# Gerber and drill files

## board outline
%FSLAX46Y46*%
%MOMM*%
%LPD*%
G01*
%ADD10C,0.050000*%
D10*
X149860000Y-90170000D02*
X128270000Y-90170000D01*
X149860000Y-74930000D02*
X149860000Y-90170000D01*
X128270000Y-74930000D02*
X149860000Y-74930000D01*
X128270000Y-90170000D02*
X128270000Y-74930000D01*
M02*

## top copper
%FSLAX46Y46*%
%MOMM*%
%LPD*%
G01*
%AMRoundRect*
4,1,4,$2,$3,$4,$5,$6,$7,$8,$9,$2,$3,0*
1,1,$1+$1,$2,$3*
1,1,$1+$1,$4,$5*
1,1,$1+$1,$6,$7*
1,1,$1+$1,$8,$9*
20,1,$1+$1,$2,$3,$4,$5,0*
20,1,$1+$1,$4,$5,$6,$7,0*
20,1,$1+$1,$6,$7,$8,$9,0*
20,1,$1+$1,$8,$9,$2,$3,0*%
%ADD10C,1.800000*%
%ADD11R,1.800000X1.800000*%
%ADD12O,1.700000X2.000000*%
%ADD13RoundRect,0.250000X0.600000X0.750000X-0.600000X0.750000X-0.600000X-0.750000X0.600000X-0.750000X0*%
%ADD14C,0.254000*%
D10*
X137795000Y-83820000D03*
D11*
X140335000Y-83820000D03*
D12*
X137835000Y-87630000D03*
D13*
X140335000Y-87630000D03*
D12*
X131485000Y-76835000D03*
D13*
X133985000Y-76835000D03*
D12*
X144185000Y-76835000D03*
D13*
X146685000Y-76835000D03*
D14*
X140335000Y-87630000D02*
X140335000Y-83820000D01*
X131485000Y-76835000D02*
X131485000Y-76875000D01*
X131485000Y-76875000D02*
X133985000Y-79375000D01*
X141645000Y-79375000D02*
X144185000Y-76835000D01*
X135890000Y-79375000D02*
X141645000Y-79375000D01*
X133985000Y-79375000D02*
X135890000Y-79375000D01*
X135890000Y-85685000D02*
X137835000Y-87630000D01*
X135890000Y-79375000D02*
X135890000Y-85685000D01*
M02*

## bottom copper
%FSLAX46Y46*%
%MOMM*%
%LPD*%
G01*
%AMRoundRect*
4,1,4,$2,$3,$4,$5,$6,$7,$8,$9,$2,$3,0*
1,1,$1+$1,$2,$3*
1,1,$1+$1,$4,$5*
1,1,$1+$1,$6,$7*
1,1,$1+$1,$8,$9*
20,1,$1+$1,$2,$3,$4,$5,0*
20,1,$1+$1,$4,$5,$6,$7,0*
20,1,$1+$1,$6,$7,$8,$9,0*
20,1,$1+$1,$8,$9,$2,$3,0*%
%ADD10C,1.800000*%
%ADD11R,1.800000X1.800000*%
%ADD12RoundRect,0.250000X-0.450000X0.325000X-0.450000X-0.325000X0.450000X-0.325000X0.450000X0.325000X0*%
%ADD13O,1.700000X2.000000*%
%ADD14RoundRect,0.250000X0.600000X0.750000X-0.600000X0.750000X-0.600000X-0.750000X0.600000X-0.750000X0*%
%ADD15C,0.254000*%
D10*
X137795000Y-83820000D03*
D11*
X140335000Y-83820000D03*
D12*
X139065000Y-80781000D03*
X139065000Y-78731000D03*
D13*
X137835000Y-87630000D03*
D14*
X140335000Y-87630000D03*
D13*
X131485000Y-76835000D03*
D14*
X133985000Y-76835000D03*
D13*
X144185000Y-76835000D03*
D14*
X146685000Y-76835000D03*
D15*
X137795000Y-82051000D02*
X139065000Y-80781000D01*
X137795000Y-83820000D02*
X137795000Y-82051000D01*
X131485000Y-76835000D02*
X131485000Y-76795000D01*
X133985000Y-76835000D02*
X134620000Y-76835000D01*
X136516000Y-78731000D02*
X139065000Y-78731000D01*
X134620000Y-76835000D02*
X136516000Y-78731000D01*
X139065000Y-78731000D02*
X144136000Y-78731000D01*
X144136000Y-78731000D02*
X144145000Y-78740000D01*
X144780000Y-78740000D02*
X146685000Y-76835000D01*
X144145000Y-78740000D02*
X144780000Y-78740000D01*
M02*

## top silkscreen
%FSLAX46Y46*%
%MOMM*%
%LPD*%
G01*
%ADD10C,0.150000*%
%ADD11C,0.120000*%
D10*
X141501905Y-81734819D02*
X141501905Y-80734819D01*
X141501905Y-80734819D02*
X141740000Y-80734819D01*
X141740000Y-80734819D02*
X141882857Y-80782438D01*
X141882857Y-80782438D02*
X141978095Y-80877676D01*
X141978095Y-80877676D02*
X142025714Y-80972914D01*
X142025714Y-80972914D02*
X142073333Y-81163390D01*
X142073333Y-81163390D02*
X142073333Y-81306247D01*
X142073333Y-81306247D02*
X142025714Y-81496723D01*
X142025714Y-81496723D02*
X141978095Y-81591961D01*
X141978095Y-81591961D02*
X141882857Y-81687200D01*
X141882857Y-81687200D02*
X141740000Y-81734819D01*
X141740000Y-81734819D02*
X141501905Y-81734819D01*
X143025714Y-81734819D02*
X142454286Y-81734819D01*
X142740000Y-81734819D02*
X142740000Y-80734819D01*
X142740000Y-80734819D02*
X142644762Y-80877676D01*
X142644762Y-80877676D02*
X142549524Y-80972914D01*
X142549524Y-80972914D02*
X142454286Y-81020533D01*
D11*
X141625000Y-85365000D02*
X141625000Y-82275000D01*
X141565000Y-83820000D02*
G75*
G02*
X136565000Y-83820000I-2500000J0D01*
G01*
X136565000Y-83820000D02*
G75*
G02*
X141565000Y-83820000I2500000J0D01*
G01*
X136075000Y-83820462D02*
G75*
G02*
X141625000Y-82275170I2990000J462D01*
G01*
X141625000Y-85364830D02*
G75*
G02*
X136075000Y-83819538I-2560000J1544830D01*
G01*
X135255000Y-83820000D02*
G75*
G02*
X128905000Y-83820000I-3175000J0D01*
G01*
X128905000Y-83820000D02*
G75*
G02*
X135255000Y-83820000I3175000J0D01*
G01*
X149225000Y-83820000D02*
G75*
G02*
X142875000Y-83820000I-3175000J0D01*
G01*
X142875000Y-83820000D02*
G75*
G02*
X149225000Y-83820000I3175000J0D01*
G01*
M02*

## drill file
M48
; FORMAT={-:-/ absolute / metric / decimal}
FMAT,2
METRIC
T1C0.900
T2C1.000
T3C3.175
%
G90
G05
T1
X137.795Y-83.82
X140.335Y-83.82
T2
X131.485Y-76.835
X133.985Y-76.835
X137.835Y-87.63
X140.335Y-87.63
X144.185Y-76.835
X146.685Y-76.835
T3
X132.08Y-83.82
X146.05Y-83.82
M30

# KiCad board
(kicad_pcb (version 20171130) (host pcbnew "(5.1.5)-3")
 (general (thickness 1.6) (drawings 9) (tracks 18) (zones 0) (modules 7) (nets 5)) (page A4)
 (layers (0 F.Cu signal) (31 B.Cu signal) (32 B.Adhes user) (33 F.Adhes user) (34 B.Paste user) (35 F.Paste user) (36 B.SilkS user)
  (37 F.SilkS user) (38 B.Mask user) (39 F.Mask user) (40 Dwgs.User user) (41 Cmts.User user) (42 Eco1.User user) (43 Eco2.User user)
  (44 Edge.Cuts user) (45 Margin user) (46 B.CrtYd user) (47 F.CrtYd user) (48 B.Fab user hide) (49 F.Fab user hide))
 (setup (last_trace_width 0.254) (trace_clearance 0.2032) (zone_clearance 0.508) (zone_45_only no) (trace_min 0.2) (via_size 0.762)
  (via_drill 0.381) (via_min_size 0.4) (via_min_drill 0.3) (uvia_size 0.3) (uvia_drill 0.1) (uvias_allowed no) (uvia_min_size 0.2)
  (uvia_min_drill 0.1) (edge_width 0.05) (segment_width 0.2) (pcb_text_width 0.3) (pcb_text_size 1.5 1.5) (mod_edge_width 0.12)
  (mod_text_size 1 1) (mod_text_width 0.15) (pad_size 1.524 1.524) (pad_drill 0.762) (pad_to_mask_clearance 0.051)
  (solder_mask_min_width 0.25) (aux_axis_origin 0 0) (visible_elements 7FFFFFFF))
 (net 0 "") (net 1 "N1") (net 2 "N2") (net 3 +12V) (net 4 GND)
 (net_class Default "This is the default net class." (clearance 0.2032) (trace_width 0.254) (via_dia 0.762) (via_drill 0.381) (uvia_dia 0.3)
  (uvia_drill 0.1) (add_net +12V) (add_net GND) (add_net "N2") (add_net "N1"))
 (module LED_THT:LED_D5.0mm (layer F.Cu) (at 140.335 83.82 180)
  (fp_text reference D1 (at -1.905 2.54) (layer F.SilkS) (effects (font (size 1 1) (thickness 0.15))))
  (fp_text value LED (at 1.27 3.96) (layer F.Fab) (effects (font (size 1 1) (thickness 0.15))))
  (fp_line (start -1.29 -1.545) (end -1.29 1.545) (layer F.SilkS) (width 0.12))
  (fp_circle (center 1.27 0) (end 3.77 0) (layer F.SilkS) (width 0.12))
  (fp_arc (start 1.27 0) (end -1.29 1.54483) (angle -148.9) (layer F.SilkS) (width 0.12))
  (fp_arc (start 1.27 0) (end -1.29 -1.54483) (angle 148.9) (layer F.SilkS) (width 0.12))
  (pad 2 thru_hole circle (at 2.54 0 180) (size 1.8 1.8) (drill 0.9) (layers *.Cu *.Mask) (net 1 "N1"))
  (pad 1 thru_hole rect (at 0 0 180) (size 1.8 1.8) (drill 0.9) (layers *.Cu *.Mask) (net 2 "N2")))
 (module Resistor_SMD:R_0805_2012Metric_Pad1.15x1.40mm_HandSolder (layer B.Cu) (at 139.065 79.756 270)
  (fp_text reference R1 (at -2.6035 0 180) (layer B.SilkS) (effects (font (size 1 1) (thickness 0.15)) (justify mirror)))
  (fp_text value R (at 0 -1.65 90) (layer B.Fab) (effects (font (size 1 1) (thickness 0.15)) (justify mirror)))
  (pad 2 smd roundrect (at 1.025 0 270) (size 1.15 1.4) (layers B.Cu B.Paste B.Mask) (roundrect_rratio 0.217391) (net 1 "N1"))
  (pad 1 smd roundrect (at -1.025 0 270) (size 1.15 1.4) (layers B.Cu B.Paste B.Mask) (roundrect_rratio 0.217391) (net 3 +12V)))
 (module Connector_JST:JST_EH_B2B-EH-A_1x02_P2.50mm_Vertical (layer B.Cu) (at 140.335 87.63 180)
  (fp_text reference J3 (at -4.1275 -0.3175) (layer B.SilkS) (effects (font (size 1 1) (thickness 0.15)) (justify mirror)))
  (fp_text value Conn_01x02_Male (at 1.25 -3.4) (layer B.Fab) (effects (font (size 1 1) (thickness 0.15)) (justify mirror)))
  (pad 2 thru_hole oval (at 2.5 0 180) (size 1.7 2) (drill 1) (layers *.Cu *.Mask) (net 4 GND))
  (pad 1 thru_hole roundrect (at 0 0 180) (size 1.7 2) (drill 1) (layers *.Cu *.Mask) (roundrect_rratio 0.147059) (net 2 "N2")))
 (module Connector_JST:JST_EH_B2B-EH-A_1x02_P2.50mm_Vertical (layer B.Cu) (at 133.985 76.835 180)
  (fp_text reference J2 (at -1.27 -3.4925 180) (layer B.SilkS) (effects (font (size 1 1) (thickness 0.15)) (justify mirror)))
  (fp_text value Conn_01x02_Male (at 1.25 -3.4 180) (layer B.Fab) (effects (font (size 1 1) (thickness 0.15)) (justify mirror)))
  (pad 2 thru_hole oval (at 2.5 0 180) (size 1.7 2) (drill 1) (layers *.Cu *.Mask) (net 4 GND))
  (pad 1 thru_hole roundrect (at 0 0 180) (size 1.7 2) (drill 1) (layers *.Cu *.Mask) (roundrect_rratio 0.147059) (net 3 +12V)))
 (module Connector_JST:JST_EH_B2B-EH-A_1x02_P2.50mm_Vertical (layer B.Cu) (at 146.685 76.835 180)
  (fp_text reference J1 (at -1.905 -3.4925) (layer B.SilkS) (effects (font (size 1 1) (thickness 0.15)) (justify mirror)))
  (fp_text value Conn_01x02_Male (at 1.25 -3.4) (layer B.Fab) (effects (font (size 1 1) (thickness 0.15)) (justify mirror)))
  (pad 2 thru_hole oval (at 2.5 0 180) (size 1.7 2) (drill 1) (layers *.Cu *.Mask) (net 4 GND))
  (pad 1 thru_hole roundrect (at 0 0 180) (size 1.7 2) (drill 1) (layers *.Cu *.Mask) (roundrect_rratio 0.147059) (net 3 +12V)))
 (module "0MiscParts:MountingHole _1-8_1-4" (layer F.Cu) (at 132.08 83.82 90)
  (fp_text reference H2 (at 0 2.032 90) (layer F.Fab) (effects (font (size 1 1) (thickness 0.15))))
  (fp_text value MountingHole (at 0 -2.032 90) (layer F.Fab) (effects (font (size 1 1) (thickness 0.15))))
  (fp_circle (center 0 0) (end 3.175 0) (layer F.SilkS) (width 0.12))
  (pad "" np_thru_hole circle (at 0 0 90) (size 3.175 3.175) (drill 3.175) (layers *.Cu *.Mask)))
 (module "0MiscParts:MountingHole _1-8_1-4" (layer F.Cu) (at 146.05 83.82)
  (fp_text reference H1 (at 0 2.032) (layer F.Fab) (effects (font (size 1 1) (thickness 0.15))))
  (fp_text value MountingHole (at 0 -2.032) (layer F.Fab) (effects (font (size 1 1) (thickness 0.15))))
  (fp_circle (center 0 0) (end 3.175 0) (layer F.SilkS) (width 0.12))
  (pad "" np_thru_hole circle (at 0 0) (size 3.175 3.175) (drill 3.175) (layers *.Cu *.Mask)))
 (gr_line (start 149.86 90.17) (end 128.27 90.17) (layer Edge.Cuts) (width 0.05))
 (gr_line (start 149.86 74.93) (end 149.86 90.17) (layer Edge.Cuts) (width 0.05))
 (gr_line (start 128.27 74.93) (end 149.86 74.93) (layer Edge.Cuts) (width 0.05))
 (gr_line (start 128.27 90.17) (end 128.27 74.93) (layer Edge.Cuts) (width 0.05))
 (segment (start 137.795 82.051) (end 139.065 80.781) (width 0.254) (layer B.Cu) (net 1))
 (segment (start 137.795 83.82) (end 137.795 82.051) (width 0.254) (layer B.Cu) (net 1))
 (segment (start 140.335 87.63) (end 140.335 83.82) (width 0.254) (layer F.Cu) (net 2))
 (segment (start 131.485 76.835) (end 131.485 76.795) (width 0.254) (layer B.Cu) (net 4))
 (segment (start 131.485 76.835) (end 131.485 76.875) (width 0.254) (layer F.Cu) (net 4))
 (segment (start 131.485 76.875) (end 133.985 79.375) (width 0.254) (layer F.Cu) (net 4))
 (segment (start 141.645 79.375) (end 144.185 76.835) (width 0.254) (layer F.Cu) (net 4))
 (segment (start 135.89 79.375) (end 141.645 79.375) (width 0.254) (layer F.Cu) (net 4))
 (segment (start 133.985 79.375) (end 135.89 79.375) (width 0.254) (layer F.Cu) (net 4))
 (segment (start 135.89 85.685) (end 137.835 87.63) (width 0.254) (layer F.Cu) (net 4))
 (segment (start 135.89 79.375) (end 135.89 85.685) (width 0.254) (layer F.Cu) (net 4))
 (segment (start 133.985 76.835) (end 134.62 76.835) (width 0.254) (layer B.Cu) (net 3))
 (segment (start 136.516 78.731) (end 139.065 78.731) (width 0.254) (layer B.Cu) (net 3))
 (segment (start 134.62 76.835) (end 136.516 78.731) (width 0.254) (layer B.Cu) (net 3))
 (segment (start 139.065 78.731) (end 144.136 78.731) (width 0.254) (layer B.Cu) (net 3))
 (segment (start 144.136 78.731) (end 144.145 78.74) (width 0.254) (layer B.Cu) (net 3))
 (segment (start 144.78 78.74) (end 146.685 76.835) (width 0.254) (layer B.Cu) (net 3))
 (segment (start 144.145 78.74) (end 144.78 78.74) (width 0.254) (layer B.Cu) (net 3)))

